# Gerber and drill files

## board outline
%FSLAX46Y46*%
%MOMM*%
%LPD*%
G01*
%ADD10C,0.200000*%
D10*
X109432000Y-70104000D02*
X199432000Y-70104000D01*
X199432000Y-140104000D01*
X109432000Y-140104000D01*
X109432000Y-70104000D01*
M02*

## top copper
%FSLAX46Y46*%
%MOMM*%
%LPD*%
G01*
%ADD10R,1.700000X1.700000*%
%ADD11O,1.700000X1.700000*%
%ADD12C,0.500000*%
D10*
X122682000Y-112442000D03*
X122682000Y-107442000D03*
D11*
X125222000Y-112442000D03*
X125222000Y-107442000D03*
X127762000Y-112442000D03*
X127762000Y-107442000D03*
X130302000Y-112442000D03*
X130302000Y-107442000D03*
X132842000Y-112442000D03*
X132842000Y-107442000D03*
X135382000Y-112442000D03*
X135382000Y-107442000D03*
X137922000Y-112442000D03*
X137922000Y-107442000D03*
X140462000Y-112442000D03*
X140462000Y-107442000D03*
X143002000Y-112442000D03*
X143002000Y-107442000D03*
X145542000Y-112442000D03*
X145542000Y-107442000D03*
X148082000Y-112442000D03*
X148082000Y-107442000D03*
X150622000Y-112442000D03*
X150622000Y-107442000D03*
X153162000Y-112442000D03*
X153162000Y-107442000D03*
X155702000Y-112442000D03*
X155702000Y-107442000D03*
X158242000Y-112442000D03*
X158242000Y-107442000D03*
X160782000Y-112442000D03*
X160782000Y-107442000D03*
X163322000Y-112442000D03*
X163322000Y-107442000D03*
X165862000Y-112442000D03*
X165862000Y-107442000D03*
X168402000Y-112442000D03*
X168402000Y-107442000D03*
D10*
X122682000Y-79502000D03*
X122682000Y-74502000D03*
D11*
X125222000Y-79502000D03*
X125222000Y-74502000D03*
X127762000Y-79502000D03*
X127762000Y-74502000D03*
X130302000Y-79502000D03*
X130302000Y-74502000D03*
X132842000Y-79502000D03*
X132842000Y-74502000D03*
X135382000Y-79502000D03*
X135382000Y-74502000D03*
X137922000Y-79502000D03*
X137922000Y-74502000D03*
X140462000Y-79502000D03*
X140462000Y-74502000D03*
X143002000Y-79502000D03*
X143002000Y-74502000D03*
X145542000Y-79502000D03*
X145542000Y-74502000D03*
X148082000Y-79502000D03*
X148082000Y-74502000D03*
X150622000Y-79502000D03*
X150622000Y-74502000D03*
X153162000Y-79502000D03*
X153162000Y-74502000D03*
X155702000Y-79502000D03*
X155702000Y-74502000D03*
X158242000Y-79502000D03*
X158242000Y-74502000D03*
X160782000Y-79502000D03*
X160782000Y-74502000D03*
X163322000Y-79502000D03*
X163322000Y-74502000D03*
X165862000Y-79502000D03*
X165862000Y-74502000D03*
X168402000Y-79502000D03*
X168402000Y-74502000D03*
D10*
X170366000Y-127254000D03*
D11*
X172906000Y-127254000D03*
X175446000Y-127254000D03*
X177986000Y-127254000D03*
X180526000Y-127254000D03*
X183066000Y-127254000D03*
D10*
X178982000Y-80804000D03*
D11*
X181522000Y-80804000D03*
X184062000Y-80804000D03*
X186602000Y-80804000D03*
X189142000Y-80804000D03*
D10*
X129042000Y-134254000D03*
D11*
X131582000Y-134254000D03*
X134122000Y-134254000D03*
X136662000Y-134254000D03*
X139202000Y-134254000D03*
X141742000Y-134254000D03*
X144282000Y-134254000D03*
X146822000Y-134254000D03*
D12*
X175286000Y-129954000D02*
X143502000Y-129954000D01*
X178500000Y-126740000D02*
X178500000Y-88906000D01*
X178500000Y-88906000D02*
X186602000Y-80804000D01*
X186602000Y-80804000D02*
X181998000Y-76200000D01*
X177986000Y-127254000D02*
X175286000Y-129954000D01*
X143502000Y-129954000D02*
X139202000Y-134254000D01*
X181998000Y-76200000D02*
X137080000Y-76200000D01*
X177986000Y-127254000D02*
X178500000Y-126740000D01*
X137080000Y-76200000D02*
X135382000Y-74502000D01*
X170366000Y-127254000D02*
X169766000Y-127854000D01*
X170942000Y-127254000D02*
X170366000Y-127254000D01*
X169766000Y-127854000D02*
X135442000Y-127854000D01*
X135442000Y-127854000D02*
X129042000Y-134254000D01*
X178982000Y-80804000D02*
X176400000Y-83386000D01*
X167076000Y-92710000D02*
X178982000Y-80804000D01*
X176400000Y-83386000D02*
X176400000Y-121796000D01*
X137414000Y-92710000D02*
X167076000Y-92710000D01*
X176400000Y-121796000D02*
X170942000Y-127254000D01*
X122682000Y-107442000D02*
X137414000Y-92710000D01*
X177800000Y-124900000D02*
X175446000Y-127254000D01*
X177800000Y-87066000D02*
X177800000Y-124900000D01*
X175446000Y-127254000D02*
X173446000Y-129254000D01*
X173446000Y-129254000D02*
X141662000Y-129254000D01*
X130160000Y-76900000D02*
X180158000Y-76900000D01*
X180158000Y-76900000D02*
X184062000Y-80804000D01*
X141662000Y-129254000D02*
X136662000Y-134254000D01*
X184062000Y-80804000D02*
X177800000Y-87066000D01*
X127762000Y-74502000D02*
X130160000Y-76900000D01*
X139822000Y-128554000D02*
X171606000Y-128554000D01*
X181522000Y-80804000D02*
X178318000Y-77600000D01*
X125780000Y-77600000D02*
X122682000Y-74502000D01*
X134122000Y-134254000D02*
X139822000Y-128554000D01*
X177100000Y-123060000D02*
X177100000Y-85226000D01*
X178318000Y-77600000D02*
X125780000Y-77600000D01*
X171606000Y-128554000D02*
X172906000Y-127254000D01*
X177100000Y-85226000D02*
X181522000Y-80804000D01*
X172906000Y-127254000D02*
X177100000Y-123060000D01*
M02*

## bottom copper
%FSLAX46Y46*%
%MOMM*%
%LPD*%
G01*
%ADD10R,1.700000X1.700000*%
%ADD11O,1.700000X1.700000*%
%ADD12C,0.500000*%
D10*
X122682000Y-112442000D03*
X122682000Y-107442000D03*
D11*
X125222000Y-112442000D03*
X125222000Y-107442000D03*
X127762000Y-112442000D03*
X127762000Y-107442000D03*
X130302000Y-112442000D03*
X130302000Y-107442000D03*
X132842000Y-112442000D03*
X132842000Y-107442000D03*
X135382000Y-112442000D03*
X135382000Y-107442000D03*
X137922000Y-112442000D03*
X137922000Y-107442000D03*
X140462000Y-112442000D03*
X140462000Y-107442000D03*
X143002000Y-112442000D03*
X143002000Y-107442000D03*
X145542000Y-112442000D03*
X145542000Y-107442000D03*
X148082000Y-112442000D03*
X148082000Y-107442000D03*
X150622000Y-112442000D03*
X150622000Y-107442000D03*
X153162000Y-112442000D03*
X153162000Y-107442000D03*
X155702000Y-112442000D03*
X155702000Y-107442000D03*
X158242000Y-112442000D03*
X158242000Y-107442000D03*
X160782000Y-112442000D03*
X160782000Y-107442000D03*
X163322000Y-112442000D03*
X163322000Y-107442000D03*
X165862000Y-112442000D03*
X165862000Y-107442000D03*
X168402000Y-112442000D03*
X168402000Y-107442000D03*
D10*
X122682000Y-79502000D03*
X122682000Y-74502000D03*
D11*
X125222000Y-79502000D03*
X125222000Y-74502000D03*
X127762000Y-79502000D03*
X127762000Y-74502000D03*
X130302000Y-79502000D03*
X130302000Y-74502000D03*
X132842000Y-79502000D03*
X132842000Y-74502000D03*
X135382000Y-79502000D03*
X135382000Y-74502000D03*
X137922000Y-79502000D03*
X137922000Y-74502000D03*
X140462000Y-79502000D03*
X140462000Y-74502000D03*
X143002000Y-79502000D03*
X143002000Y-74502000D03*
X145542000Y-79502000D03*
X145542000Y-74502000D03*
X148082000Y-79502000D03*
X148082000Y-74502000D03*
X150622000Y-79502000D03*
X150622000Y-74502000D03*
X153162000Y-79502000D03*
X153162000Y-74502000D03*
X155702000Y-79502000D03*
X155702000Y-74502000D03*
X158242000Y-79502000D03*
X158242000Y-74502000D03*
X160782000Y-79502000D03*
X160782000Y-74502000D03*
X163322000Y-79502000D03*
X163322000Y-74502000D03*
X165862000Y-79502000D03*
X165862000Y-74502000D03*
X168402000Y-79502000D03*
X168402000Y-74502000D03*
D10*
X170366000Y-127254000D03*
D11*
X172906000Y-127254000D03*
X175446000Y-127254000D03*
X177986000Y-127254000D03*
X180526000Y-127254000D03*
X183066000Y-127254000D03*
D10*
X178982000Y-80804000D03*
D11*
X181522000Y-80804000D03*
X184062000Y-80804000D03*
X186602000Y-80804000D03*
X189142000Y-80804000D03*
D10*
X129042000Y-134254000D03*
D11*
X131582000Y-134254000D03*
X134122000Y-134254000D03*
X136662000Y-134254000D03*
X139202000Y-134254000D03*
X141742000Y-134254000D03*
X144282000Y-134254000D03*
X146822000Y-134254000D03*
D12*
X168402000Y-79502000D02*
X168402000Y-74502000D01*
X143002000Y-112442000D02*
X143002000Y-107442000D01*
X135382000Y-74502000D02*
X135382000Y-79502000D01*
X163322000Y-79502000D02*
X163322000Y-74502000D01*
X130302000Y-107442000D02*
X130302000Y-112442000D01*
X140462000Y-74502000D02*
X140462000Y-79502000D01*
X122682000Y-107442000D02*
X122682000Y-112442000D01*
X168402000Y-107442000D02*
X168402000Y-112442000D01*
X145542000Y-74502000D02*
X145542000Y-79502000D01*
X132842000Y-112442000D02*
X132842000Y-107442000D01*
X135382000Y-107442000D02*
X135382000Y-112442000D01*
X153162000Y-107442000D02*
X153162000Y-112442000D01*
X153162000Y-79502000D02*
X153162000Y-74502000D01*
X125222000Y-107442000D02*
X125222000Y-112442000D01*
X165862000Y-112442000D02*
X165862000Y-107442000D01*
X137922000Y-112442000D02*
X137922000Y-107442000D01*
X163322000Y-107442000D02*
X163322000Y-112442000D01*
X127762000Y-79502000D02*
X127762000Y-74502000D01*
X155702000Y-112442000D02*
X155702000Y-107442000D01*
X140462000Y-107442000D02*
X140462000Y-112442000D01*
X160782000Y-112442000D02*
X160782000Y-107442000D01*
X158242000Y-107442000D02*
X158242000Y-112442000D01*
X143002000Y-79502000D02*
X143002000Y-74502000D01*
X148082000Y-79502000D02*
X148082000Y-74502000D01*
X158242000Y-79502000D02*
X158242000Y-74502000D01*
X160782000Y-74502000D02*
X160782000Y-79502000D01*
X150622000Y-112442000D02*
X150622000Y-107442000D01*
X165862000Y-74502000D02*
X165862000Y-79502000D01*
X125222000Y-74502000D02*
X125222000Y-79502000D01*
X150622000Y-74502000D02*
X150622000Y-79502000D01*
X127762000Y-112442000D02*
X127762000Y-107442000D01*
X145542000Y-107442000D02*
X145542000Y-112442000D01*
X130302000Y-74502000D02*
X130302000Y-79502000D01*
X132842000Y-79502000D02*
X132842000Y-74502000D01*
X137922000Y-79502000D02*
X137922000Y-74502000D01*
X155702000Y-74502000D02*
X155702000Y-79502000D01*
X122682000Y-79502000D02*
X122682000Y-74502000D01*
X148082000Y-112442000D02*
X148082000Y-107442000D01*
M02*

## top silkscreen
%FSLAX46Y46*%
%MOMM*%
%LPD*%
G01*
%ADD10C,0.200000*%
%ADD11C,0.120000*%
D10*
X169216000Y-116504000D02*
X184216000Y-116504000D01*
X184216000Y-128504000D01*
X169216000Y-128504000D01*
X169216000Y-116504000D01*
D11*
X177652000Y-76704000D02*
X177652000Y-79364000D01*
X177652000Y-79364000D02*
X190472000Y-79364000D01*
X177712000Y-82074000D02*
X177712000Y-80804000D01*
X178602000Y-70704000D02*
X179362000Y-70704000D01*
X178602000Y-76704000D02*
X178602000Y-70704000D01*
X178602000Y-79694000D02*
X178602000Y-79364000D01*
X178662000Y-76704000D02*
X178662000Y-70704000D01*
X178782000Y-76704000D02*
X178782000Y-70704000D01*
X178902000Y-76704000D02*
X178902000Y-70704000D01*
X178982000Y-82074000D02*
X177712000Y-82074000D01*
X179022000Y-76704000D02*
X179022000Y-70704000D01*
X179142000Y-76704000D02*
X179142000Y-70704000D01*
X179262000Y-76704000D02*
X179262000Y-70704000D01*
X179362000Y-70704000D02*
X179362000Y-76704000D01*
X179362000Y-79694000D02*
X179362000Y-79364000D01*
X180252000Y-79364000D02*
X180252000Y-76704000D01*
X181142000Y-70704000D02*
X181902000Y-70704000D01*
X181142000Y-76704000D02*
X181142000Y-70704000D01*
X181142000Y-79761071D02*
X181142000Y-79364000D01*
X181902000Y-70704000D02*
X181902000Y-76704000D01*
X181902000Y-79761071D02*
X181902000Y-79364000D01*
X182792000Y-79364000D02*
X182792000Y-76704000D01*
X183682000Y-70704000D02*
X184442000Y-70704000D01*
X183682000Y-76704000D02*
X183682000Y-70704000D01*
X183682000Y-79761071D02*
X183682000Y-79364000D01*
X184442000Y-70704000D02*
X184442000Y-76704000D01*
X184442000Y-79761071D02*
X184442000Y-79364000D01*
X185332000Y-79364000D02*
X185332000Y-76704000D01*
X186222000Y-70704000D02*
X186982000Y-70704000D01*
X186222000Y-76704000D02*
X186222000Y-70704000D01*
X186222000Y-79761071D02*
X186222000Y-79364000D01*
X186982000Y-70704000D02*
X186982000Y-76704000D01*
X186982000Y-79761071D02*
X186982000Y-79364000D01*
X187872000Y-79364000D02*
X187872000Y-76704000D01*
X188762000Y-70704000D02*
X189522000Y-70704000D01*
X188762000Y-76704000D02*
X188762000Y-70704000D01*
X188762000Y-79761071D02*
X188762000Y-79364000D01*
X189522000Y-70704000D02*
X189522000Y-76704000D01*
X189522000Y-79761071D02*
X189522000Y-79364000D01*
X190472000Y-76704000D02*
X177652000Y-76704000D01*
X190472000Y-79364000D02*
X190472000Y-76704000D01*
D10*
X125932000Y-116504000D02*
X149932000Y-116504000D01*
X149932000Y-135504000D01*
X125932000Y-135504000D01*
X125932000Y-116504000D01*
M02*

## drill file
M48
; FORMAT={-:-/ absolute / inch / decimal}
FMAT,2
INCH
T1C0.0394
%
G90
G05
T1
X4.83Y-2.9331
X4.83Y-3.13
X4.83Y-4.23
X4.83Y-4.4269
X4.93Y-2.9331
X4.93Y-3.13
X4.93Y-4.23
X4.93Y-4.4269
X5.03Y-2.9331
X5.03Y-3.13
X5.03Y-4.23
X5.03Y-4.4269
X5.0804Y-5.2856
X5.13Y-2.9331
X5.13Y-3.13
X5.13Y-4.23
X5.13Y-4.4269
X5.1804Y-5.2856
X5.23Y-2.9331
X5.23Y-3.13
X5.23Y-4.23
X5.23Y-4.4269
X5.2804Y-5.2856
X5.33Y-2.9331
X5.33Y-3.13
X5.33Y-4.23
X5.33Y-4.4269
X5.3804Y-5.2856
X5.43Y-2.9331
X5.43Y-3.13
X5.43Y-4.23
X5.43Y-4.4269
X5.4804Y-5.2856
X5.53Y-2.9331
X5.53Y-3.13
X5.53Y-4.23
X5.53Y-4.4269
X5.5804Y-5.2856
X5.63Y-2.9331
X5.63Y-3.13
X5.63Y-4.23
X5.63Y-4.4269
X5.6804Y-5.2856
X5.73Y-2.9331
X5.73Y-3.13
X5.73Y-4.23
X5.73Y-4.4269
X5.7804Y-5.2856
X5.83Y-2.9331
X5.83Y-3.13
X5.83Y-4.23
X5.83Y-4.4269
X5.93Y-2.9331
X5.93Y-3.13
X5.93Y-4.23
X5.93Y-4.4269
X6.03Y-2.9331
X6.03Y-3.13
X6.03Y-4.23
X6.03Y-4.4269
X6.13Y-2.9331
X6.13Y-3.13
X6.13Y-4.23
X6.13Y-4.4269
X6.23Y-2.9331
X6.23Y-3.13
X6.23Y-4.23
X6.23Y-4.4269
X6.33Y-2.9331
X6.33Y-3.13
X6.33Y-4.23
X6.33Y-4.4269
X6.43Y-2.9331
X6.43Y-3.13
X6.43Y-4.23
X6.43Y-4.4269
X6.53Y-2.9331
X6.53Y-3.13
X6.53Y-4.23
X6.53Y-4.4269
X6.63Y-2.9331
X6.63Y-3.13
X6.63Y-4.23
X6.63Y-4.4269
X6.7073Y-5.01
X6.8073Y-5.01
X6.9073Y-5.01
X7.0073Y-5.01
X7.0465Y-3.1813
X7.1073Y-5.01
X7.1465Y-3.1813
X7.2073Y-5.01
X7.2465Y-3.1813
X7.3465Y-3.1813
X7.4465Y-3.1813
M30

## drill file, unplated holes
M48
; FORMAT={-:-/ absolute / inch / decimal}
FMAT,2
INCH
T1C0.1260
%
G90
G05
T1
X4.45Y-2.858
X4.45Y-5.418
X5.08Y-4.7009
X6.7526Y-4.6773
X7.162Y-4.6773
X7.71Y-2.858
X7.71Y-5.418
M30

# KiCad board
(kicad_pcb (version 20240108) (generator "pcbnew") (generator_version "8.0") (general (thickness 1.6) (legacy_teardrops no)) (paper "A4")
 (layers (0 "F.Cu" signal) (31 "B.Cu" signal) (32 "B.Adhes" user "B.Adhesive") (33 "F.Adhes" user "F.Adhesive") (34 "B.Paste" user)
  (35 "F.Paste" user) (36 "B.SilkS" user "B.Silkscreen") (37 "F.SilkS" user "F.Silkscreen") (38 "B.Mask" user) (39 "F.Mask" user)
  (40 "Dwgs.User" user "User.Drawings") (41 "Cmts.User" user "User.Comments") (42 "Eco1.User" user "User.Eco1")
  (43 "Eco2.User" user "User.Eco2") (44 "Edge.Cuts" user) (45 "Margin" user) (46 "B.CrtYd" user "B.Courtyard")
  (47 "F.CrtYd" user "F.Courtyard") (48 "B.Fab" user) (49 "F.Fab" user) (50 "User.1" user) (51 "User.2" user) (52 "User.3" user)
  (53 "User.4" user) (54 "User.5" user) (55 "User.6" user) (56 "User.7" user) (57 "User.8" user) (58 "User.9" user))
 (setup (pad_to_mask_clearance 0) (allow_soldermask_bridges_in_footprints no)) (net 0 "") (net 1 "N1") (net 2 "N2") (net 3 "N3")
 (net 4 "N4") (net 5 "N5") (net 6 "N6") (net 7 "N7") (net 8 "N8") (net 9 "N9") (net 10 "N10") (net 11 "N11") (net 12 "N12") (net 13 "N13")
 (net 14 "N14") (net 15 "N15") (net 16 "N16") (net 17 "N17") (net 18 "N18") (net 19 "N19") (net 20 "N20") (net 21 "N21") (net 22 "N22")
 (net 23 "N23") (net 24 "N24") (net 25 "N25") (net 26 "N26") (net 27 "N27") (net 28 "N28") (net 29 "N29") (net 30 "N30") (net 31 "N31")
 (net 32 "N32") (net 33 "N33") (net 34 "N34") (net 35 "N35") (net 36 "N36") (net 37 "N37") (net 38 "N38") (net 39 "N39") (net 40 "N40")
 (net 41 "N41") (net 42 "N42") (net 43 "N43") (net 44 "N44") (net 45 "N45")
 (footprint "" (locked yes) (layer "F.Cu") (at 113.03 72.592)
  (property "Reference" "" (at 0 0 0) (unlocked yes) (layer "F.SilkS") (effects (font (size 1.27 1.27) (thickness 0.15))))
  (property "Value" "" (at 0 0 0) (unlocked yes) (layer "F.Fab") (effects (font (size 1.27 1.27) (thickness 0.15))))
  (pad "" np_thru_hole circle (at 0 0) (size 3.2 3.2) (drill 3.2) (layers "F&B.Cu" "*.Mask")))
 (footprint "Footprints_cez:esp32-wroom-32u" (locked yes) (layer "F.Cu") (at 134.864 94.742 90)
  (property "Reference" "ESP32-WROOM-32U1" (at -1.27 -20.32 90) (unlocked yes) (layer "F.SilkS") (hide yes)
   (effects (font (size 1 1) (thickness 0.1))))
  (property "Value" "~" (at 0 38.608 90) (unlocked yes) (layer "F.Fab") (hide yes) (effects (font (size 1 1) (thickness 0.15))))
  (pad "1" thru_hole rect (at -17.7 -12.182 90) (size 1.7 1.7) (drill 1) (layers "*.Cu" "*.Mask") (remove_unused_layers no) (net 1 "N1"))
  (pad "1" thru_hole rect (at -12.7 -12.182 90) (size 1.7 1.7) (drill 1) (layers "*.Cu" "*.Mask") (remove_unused_layers no) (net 1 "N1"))
  (pad "2" thru_hole oval (at -17.7 -9.642 90) (size 1.7 1.7) (drill 1) (layers "*.Cu" "*.Mask") (remove_unused_layers no) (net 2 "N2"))
  (pad "2" thru_hole oval (at -12.7 -9.642 90) (size 1.7 1.7) (drill 1) (layers "*.Cu" "*.Mask") (remove_unused_layers no) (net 2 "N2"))
  (pad "3" thru_hole oval (at -17.7 -7.102 90) (size 1.7 1.7) (drill 1) (layers "*.Cu" "*.Mask") (remove_unused_layers no) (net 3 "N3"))
  (pad "3" thru_hole oval (at -12.7 -7.102 90) (size 1.7 1.7) (drill 1) (layers "*.Cu" "*.Mask") (remove_unused_layers no) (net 3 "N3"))
  (pad "4" thru_hole oval (at -17.7 -4.562 90) (size 1.7 1.7) (drill 1) (layers "*.Cu" "*.Mask") (remove_unused_layers no) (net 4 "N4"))
  (pad "4" thru_hole oval (at -12.7 -4.562 90) (size 1.7 1.7) (drill 1) (layers "*.Cu" "*.Mask") (remove_unused_layers no) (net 4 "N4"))
  (pad "5" thru_hole oval (at -17.7 -2.022 90) (size 1.7 1.7) (drill 1) (layers "*.Cu" "*.Mask") (remove_unused_layers no) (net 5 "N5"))
  (pad "5" thru_hole oval (at -12.7 -2.022 90) (size 1.7 1.7) (drill 1) (layers "*.Cu" "*.Mask") (remove_unused_layers no) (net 5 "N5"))
  (pad "6" thru_hole oval (at -17.7 0.518 90) (size 1.7 1.7) (drill 1) (layers "*.Cu" "*.Mask") (remove_unused_layers no) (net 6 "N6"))
  (pad "6" thru_hole oval (at -12.7 0.518 90) (size 1.7 1.7) (drill 1) (layers "*.Cu" "*.Mask") (remove_unused_layers no) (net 6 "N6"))
  (pad "7" thru_hole oval (at -17.7 3.058 90) (size 1.7 1.7) (drill 1) (layers "*.Cu" "*.Mask") (remove_unused_layers no) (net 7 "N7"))
  (pad "7" thru_hole oval (at -12.7 3.058 90) (size 1.7 1.7) (drill 1) (layers "*.Cu" "*.Mask") (remove_unused_layers no) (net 7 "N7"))
  (pad "8" thru_hole oval (at -17.7 5.598 90) (size 1.7 1.7) (drill 1) (layers "*.Cu" "*.Mask") (remove_unused_layers no) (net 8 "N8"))
  (pad "8" thru_hole oval (at -12.7 5.598 90) (size 1.7 1.7) (drill 1) (layers "*.Cu" "*.Mask") (remove_unused_layers no) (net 8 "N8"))
  (pad "9" thru_hole oval (at -17.7 8.138 90) (size 1.7 1.7) (drill 1) (layers "*.Cu" "*.Mask") (remove_unused_layers no) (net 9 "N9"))
  (pad "9" thru_hole oval (at -12.7 8.138 90) (size 1.7 1.7) (drill 1) (layers "*.Cu" "*.Mask") (remove_unused_layers no) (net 9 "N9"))
  (pad "10" thru_hole oval (at -17.7 10.678 90) (size 1.7 1.7) (drill 1) (layers "*.Cu" "*.Mask") (remove_unused_layers no) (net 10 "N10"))
  (pad "10" thru_hole oval (at -12.7 10.678 90) (size 1.7 1.7) (drill 1) (layers "*.Cu" "*.Mask") (remove_unused_layers no) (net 10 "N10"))
  (pad "11" thru_hole oval (at -17.7 13.218 90) (size 1.7 1.7) (drill 1) (layers "*.Cu" "*.Mask") (remove_unused_layers no) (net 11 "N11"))
  (pad "11" thru_hole oval (at -12.7 13.218 90) (size 1.7 1.7) (drill 1) (layers "*.Cu" "*.Mask") (remove_unused_layers no) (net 11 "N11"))
  (pad "12" thru_hole oval (at -17.7 15.758 90) (size 1.7 1.7) (drill 1) (layers "*.Cu" "*.Mask") (remove_unused_layers no) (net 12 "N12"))
  (pad "12" thru_hole oval (at -12.7 15.758 90) (size 1.7 1.7) (drill 1) (layers "*.Cu" "*.Mask") (remove_unused_layers no) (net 12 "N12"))
  (pad "13" thru_hole oval (at -17.7 18.298 90) (size 1.7 1.7) (drill 1) (layers "*.Cu" "*.Mask") (remove_unused_layers no) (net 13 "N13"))
  (pad "13" thru_hole oval (at -12.7 18.298 90) (size 1.7 1.7) (drill 1) (layers "*.Cu" "*.Mask") (remove_unused_layers no) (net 13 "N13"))
  (pad "14" thru_hole oval (at -17.7 20.838 90) (size 1.7 1.7) (drill 1) (layers "*.Cu" "*.Mask") (remove_unused_layers no) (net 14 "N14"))
  (pad "14" thru_hole oval (at -12.7 20.838 90) (size 1.7 1.7) (drill 1) (layers "*.Cu" "*.Mask") (remove_unused_layers no) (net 14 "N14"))
  (pad "15" thru_hole oval (at -17.7 23.378 90) (size 1.7 1.7) (drill 1) (layers "*.Cu" "*.Mask") (remove_unused_layers no) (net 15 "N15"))
  (pad "15" thru_hole oval (at -12.7 23.378 90) (size 1.7 1.7) (drill 1) (layers "*.Cu" "*.Mask") (remove_unused_layers no) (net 15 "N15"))
  (pad "16" thru_hole oval (at -17.7 25.918 90) (size 1.7 1.7) (drill 1) (layers "*.Cu" "*.Mask") (remove_unused_layers no) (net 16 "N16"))
  (pad "16" thru_hole oval (at -12.7 25.918 90) (size 1.7 1.7) (drill 1) (layers "*.Cu" "*.Mask") (remove_unused_layers no) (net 16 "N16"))
  (pad "17" thru_hole oval (at -17.7 28.458 90) (size 1.7 1.7) (drill 1) (layers "*.Cu" "*.Mask") (remove_unused_layers no) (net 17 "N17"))
  (pad "17" thru_hole oval (at -12.7 28.458 90) (size 1.7 1.7) (drill 1) (layers "*.Cu" "*.Mask") (remove_unused_layers no) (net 17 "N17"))
  (pad "18" thru_hole oval (at -17.7 30.998 90) (size 1.7 1.7) (drill 1) (layers "*.Cu" "*.Mask") (remove_unused_layers no) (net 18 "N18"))
  (pad "18" thru_hole oval (at -12.7 30.998 90) (size 1.7 1.7) (drill 1) (layers "*.Cu" "*.Mask") (remove_unused_layers no) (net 18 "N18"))
  (pad "19" thru_hole oval (at -17.7 33.538 90) (size 1.7 1.7) (drill 1) (layers "*.Cu" "*.Mask") (remove_unused_layers no) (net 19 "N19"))
  (pad "19" thru_hole oval (at -12.7 33.538 90) (size 1.7 1.7) (drill 1) (layers "*.Cu" "*.Mask") (remove_unused_layers no) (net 19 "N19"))
  (pad "20" thru_hole rect (at 15.24 -12.182 90) (size 1.7 1.7) (drill 1) (layers "*.Cu" "*.Mask") (remove_unused_layers no) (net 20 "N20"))
  (pad "20" thru_hole rect (at 20.24 -12.182 90) (size 1.7 1.7) (drill 1) (layers "*.Cu" "*.Mask") (remove_unused_layers no) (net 20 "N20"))
  (pad "21" thru_hole oval (at 15.24 -9.642 90) (size 1.7 1.7) (drill 1) (layers "*.Cu" "*.Mask") (remove_unused_layers no) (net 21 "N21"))
  (pad "21" thru_hole oval (at 20.24 -9.642 90) (size 1.7 1.7) (drill 1) (layers "*.Cu" "*.Mask") (remove_unused_layers no) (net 21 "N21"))
  (pad "22" thru_hole oval (at 15.24 -7.102 90) (size 1.7 1.7) (drill 1) (layers "*.Cu" "*.Mask") (remove_unused_layers no) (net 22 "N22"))
  (pad "22" thru_hole oval (at 20.24 -7.102 90) (size 1.7 1.7) (drill 1) (layers "*.Cu" "*.Mask") (remove_unused_layers no) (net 22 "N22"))
  (pad "23" thru_hole oval (at 15.24 -4.562 90) (size 1.7 1.7) (drill 1) (layers "*.Cu" "*.Mask") (remove_unused_layers no) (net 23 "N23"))
  (pad "23" thru_hole oval (at 20.24 -4.562 90) (size 1.7 1.7) (drill 1) (layers "*.Cu" "*.Mask") (remove_unused_layers no) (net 23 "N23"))
  (pad "24" thru_hole oval (at 15.24 -2.022 90) (size 1.7 1.7) (drill 1) (layers "*.Cu" "*.Mask") (remove_unused_layers no) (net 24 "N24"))
  (pad "24" thru_hole oval (at 20.24 -2.022 90) (size 1.7 1.7) (drill 1) (layers "*.Cu" "*.Mask") (remove_unused_layers no) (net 24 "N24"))
  (pad "25" thru_hole oval (at 15.24 0.518 90) (size 1.7 1.7) (drill 1) (layers "*.Cu" "*.Mask") (remove_unused_layers no) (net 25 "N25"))
  (pad "25" thru_hole oval (at 20.24 0.518 90) (size 1.7 1.7) (drill 1) (layers "*.Cu" "*.Mask") (remove_unused_layers no) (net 25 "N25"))
  (pad "26" thru_hole oval (at 15.24 3.058 90) (size 1.7 1.7) (drill 1) (layers "*.Cu" "*.Mask") (remove_unused_layers no) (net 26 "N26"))
  (pad "26" thru_hole oval (at 20.24 3.058 90) (size 1.7 1.7) (drill 1) (layers "*.Cu" "*.Mask") (remove_unused_layers no) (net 26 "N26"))
  (pad "27" thru_hole oval (at 15.24 5.598 90) (size 1.7 1.7) (drill 1) (layers "*.Cu" "*.Mask") (remove_unused_layers no) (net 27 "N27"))
  (pad "27" thru_hole oval (at 20.24 5.598 90) (size 1.7 1.7) (drill 1) (layers "*.Cu" "*.Mask") (remove_unused_layers no) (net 27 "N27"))
  (pad "28" thru_hole oval (at 15.24 8.138 90) (size 1.7 1.7) (drill 1) (layers "*.Cu" "*.Mask") (remove_unused_layers no) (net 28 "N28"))
  (pad "28" thru_hole oval (at 20.24 8.138 90) (size 1.7 1.7) (drill 1) (layers "*.Cu" "*.Mask") (remove_unused_layers no) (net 28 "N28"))
  (pad "29" thru_hole oval (at 15.24 10.678 90) (size 1.7 1.7) (drill 1) (layers "*.Cu" "*.Mask") (remove_unused_layers no) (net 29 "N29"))
  (pad "29" thru_hole oval (at 20.24 10.678 90) (size 1.7 1.7) (drill 1) (layers "*.Cu" "*.Mask") (remove_unused_layers no) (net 29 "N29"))
  (pad "30" thru_hole oval (at 15.24 13.218 90) (size 1.7 1.7) (drill 1) (layers "*.Cu" "*.Mask") (remove_unused_layers no) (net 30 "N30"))
  (pad "30" thru_hole oval (at 20.24 13.218 90) (size 1.7 1.7) (drill 1) (layers "*.Cu" "*.Mask") (remove_unused_layers no) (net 30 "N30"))
  (pad "31" thru_hole oval (at 15.24 15.758 90) (size 1.7 1.7) (drill 1) (layers "*.Cu" "*.Mask") (remove_unused_layers no) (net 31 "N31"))
  (pad "31" thru_hole oval (at 20.24 15.758 90) (size 1.7 1.7) (drill 1) (layers "*.Cu" "*.Mask") (remove_unused_layers no) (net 31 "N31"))
  (pad "32" thru_hole oval (at 15.24 18.298 90) (size 1.7 1.7) (drill 1) (layers "*.Cu" "*.Mask") (remove_unused_layers no) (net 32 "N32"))
  (pad "32" thru_hole oval (at 20.24 18.298 90) (size 1.7 1.7) (drill 1) (layers "*.Cu" "*.Mask") (remove_unused_layers no) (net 32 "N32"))
  (pad "33" thru_hole oval (at 15.24 20.838 90) (size 1.7 1.7) (drill 1) (layers "*.Cu" "*.Mask") (remove_unused_layers no) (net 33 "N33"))
  (pad "33" thru_hole oval (at 20.24 20.838 90) (size 1.7 1.7) (drill 1) (layers "*.Cu" "*.Mask") (remove_unused_layers no) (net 33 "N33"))
  (pad "34" thru_hole oval (at 15.24 23.378 90) (size 1.7 1.7) (drill 1) (layers "*.Cu" "*.Mask") (remove_unused_layers no) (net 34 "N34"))
  (pad "34" thru_hole oval (at 20.24 23.378 90) (size 1.7 1.7) (drill 1) (layers "*.Cu" "*.Mask") (remove_unused_layers no) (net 34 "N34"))
  (pad "35" thru_hole oval (at 15.24 25.918 90) (size 1.7 1.7) (drill 1) (layers "*.Cu" "*.Mask") (remove_unused_layers no) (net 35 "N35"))
  (pad "35" thru_hole oval (at 20.24 25.918 90) (size 1.7 1.7) (drill 1) (layers "*.Cu" "*.Mask") (remove_unused_layers no) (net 35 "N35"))
  (pad "36" thru_hole oval (at 15.24 28.458 90) (size 1.7 1.7) (drill 1) (layers "*.Cu" "*.Mask") (remove_unused_layers no) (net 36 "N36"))
  (pad "36" thru_hole oval (at 20.24 28.458 90) (size 1.7 1.7) (drill 1) (layers "*.Cu" "*.Mask") (remove_unused_layers no) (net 36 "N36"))
  (pad "37" thru_hole oval (at 15.24 30.998 90) (size 1.7 1.7) (drill 1) (layers "*.Cu" "*.Mask") (remove_unused_layers no) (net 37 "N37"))
  (pad "37" thru_hole oval (at 20.24 30.998 90) (size 1.7 1.7) (drill 1) (layers "*.Cu" "*.Mask") (remove_unused_layers no) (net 37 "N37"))
  (pad "38" thru_hole oval (at 15.24 33.538 90) (size 1.7 1.7) (drill 1) (layers "*.Cu" "*.Mask") (remove_unused_layers no) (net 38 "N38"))
  (pad "38" thru_hole oval (at 20.24 33.538 90) (size 1.7 1.7) (drill 1) (layers "*.Cu" "*.Mask") (remove_unused_layers no) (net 38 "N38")))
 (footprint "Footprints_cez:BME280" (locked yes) (layer "F.Cu") (at 178.755 110.185)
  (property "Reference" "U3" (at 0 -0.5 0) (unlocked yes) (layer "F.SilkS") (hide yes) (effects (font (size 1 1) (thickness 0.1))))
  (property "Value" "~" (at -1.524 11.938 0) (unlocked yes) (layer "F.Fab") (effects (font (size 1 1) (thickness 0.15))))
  (fp_rect (start -9.539 6.319) (end 5.461 18.319) (stroke (width 0.2) (type default)) (fill none) (layer "F.SilkS"))
  (pad "" np_thru_hole circle (at -7.239 8.619) (size 3.2 3.2) (drill 3.2) (layers "F&B.Cu" "*.Mask"))
  (pad "" np_thru_hole circle (at 3.161 8.619) (size 3.2 3.2) (drill 3.2) (layers "F&B.Cu" "*.Mask"))
  (pad "1" thru_hole rect (at -8.389 17.069 90) (size 1.7 1.7) (drill 1) (layers "*.Cu" "*.Mask") (remove_unused_layers no) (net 1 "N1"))
  (pad "2" thru_hole oval (at -5.849 17.069 90) (size 1.7 1.7) (drill 1) (layers "*.Cu" "*.Mask") (remove_unused_layers no) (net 20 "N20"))
  (pad "3" thru_hole oval (at -3.309 17.069 90) (size 1.7 1.7) (drill 1) (layers "*.Cu" "*.Mask") (remove_unused_layers no) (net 22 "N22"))
  (pad "4" thru_hole oval (at -0.769 17.069 90) (size 1.7 1.7) (drill 1) (layers "*.Cu" "*.Mask") (remove_unused_layers no) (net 25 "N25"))
  (pad "5" thru_hole oval (at 1.771 17.069 90) (size 1.7 1.7) (drill 1) (layers "*.Cu" "*.Mask") (remove_unused_layers no) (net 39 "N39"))
  (pad "6" thru_hole oval (at 4.311 17.069 90) (size 1.7 1.7) (drill 1) (layers "*.Cu" "*.Mask") (remove_unused_layers no) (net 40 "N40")))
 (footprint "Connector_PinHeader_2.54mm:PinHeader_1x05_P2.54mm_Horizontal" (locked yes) (layer "F.Cu") (at 178.982 80.804 90)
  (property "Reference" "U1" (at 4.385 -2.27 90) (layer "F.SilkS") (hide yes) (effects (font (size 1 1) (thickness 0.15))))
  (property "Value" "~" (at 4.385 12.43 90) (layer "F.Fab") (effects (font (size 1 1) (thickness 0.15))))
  (fp_line (start 4.1 -1.33) (end 1.44 -1.33) (stroke (width 0.12) (type solid)) (layer "F.SilkS"))
  (fp_line (start 1.44 -1.33) (end 1.44 11.49) (stroke (width 0.12) (type solid)) (layer "F.SilkS"))
  (fp_line (start -1.27 -1.27) (end 0 -1.27) (stroke (width 0.12) (type solid)) (layer "F.SilkS"))
  (fp_line (start 10.1 -0.38) (end 10.1 0.38) (stroke (width 0.12) (type solid)) (layer "F.SilkS"))
  (fp_line (start 4.1 -0.38) (end 10.1 -0.38) (stroke (width 0.12) (type solid)) (layer "F.SilkS"))
  (fp_line (start 1.11 -0.38) (end 1.44 -0.38) (stroke (width 0.12) (type solid)) (layer "F.SilkS"))
  (fp_line (start 4.1 -0.32) (end 10.1 -0.32) (stroke (width 0.12) (type solid)) (layer "F.SilkS"))
  (fp_line (start 4.1 -0.2) (end 10.1 -0.2) (stroke (width 0.12) (type solid)) (layer "F.SilkS"))
  (fp_line (start 4.1 -0.08) (end 10.1 -0.08) (stroke (width 0.12) (type solid)) (layer "F.SilkS"))
  (fp_line (start -1.27 0) (end -1.27 -1.27) (stroke (width 0.12) (type solid)) (layer "F.SilkS"))
  (fp_line (start 4.1 0.04) (end 10.1 0.04) (stroke (width 0.12) (type solid)) (layer "F.SilkS"))
  (fp_line (start 4.1 0.16) (end 10.1 0.16) (stroke (width 0.12) (type solid)) (layer "F.SilkS"))
  (fp_line (start 4.1 0.28) (end 10.1 0.28) (stroke (width 0.12) (type solid)) (layer "F.SilkS"))
  (fp_line (start 10.1 0.38) (end 4.1 0.38) (stroke (width 0.12) (type solid)) (layer "F.SilkS"))
  (fp_line (start 1.11 0.38) (end 1.44 0.38) (stroke (width 0.12) (type solid)) (layer "F.SilkS"))
  (fp_line (start 1.44 1.27) (end 4.1 1.27) (stroke (width 0.12) (type solid)) (layer "F.SilkS"))
  (fp_line (start 10.1 2.16) (end 10.1 2.92) (stroke (width 0.12) (type solid)) (layer "F.SilkS"))
  (fp_line (start 4.1 2.16) (end 10.1 2.16) (stroke (width 0.12) (type solid)) (layer "F.SilkS"))
  (fp_line (start 1.042929 2.16) (end 1.44 2.16) (stroke (width 0.12) (type solid)) (layer "F.SilkS"))
  (fp_line (start 10.1 2.92) (end 4.1 2.92) (stroke (width 0.12) (type solid)) (layer "F.SilkS"))
  (fp_line (start 1.042929 2.92) (end 1.44 2.92) (stroke (width 0.12) (type solid)) (layer "F.SilkS"))
  (fp_line (start 1.44 3.81) (end 4.1 3.81) (stroke (width 0.12) (type solid)) (layer "F.SilkS"))
  (fp_line (start 10.1 4.7) (end 10.1 5.46) (stroke (width 0.12) (type solid)) (layer "F.SilkS"))
  (fp_line (start 4.1 4.7) (end 10.1 4.7) (stroke (width 0.12) (type solid)) (layer "F.SilkS"))
  (fp_line (start 1.042929 4.7) (end 1.44 4.7) (stroke (width 0.12) (type solid)) (layer "F.SilkS"))
  (fp_line (start 10.1 5.46) (end 4.1 5.46) (stroke (width 0.12) (type solid)) (layer "F.SilkS"))
  (fp_line (start 1.042929 5.46) (end 1.44 5.46) (stroke (width 0.12) (type solid)) (layer "F.SilkS"))
  (fp_line (start 1.44 6.35) (end 4.1 6.35) (stroke (width 0.12) (type solid)) (layer "F.SilkS"))
  (fp_line (start 10.1 7.24) (end 10.1 8) (stroke (width 0.12) (type solid)) (layer "F.SilkS"))
  (fp_line (start 4.1 7.24) (end 10.1 7.24) (stroke (width 0.12) (type solid)) (layer "F.SilkS"))
  (fp_line (start 1.042929 7.24) (end 1.44 7.24) (stroke (width 0.12) (type solid)) (layer "F.SilkS"))
  (fp_line (start 10.1 8) (end 4.1 8) (stroke (width 0.12) (type solid)) (layer "F.SilkS"))
  (fp_line (start 1.042929 8) (end 1.44 8) (stroke (width 0.12) (type solid)) (layer "F.SilkS"))
  (fp_line (start 1.44 8.89) (end 4.1 8.89) (stroke (width 0.12) (type solid)) (layer "F.SilkS"))
  (fp_line (start 10.1 9.78) (end 10.1 10.54) (stroke (width 0.12) (type solid)) (layer "F.SilkS"))
  (fp_line (start 4.1 9.78) (end 10.1 9.78) (stroke (width 0.12) (type solid)) (layer "F.SilkS"))
  (fp_line (start 1.042929 9.78) (end 1.44 9.78) (stroke (width 0.12) (type solid)) (layer "F.SilkS"))
  (fp_line (start 10.1 10.54) (end 4.1 10.54) (stroke (width 0.12) (type solid)) (layer "F.SilkS"))
  (fp_line (start 1.042929 10.54) (end 1.44 10.54) (stroke (width 0.12) (type solid)) (layer "F.SilkS"))
  (fp_line (start 4.1 11.49) (end 4.1 -1.33) (stroke (width 0.12) (type solid)) (layer "F.SilkS"))
  (fp_line (start 1.44 11.49) (end 4.1 11.49) (stroke (width 0.12) (type solid)) (layer "F.SilkS"))
  (pad "1" thru_hole rect (at 0 0 90) (size 1.7 1.7) (drill 1) (layers "*.Cu" "*.Mask") (remove_unused_layers no) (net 1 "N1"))
  (pad "2" thru_hole oval (at 0 2.54 90) (size 1.7 1.7) (drill 1) (layers "*.Cu" "*.Mask") (remove_unused_layers no) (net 20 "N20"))
  (pad "3" thru_hole oval (at 0 5.08 90) (size 1.7 1.7) (drill 1) (layers "*.Cu" "*.Mask") (remove_unused_layers no) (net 22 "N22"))
  (pad "4" thru_hole oval (at 0 7.62 90) (size 1.7 1.7) (drill 1) (layers "*.Cu" "*.Mask") (remove_unused_layers no) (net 25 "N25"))
  (pad "5" thru_hole oval (at 0 10.16 90) (size 1.7 1.7) (drill 1) (layers "*.Cu" "*.Mask") (remove_unused_layers no) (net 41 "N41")))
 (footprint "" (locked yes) (layer "F.Cu") (at 113.03 137.616)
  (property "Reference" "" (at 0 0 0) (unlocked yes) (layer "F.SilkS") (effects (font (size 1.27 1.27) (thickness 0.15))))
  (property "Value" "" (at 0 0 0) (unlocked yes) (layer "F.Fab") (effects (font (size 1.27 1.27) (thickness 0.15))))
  (pad "" np_thru_hole circle (at 0 0) (size 3.2 3.2) (drill 3.2) (layers "F&B.Cu" "*.Mask")))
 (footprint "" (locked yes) (layer "F.Cu") (at 195.834 137.616)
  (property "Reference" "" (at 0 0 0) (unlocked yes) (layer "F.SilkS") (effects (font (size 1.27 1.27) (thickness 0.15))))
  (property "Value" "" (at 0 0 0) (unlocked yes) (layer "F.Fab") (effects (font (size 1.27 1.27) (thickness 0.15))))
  (pad "" np_thru_hole circle (at 0 0) (size 3.2 3.2) (drill 3.2) (layers "F&B.Cu" "*.Mask")))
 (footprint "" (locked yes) (layer "F.Cu") (at 195.834 72.592)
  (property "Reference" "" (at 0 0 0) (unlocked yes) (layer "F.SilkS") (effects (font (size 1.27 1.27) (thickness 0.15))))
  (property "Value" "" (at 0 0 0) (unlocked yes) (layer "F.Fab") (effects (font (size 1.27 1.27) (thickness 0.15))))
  (pad "" np_thru_hole circle (at 0 0) (size 3.2 3.2) (drill 3.2) (layers "F&B.Cu" "*.Mask")))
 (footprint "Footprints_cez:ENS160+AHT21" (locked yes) (layer "F.Cu") (at 136.027 102.611)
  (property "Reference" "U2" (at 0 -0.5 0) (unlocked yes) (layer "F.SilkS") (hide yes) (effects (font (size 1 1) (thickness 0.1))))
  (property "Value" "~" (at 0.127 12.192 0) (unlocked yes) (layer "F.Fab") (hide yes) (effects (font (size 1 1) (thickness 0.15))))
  (fp_rect (start -10.095 13.893) (end 13.905 32.893) (stroke (width 0.2) (type default)) (fill none) (layer "F.SilkS"))
  (pad "" np_thru_hole circle (at -6.995 16.793) (size 3.2 3.2) (drill 3.2) (layers "*.Cu" "*.Mask"))
  (pad "1" thru_hole rect (at -6.985 31.643 90) (size 1.7 1.7) (drill 1) (layers "*.Cu" "*.Mask") (remove_unused_layers no) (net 1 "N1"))
  (pad "2" thru_hole oval (at -4.445 31.643 90) (size 1.7 1.7) (drill 1) (layers "*.Cu" "*.Mask") (remove_unused_layers no) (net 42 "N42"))
  (pad "3" thru_hole oval (at -1.905 31.643 90) (size 1.7 1.7) (drill 1) (layers "*.Cu" "*.Mask") (remove_unused_layers no) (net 20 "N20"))
  (pad "4" thru_hole oval (at 0.635 31.643 90) (size 1.7 1.7) (drill 1) (layers "*.Cu" "*.Mask") (remove_unused_layers no) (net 22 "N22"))
  (pad "5" thru_hole oval (at 3.175 31.643 90) (size 1.7 1.7) (drill 1) (layers "*.Cu" "*.Mask") (remove_unused_layers no) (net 25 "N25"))
  (pad "6" thru_hole oval (at 5.715 31.643 90) (size 1.7 1.7) (drill 1) (layers "*.Cu" "*.Mask") (remove_unused_layers no) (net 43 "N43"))
  (pad "7" thru_hole oval (at 8.255 31.643 90) (size 1.7 1.7) (drill 1) (layers "*.Cu" "*.Mask") (remove_unused_layers no) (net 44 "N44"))
  (pad "8" thru_hole oval (at 10.795 31.643 90) (size 1.7 1.7) (drill 1) (layers "*.Cu" "*.Mask") (remove_unused_layers no) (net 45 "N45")))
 (gr_rect (start 109.432 70.104) (end 199.432 140.104) (locked yes) (stroke (width 0.2) (type default)) (fill none) (layer "Edge.Cuts"))
 (segment (start 168.402 79.502) (end 168.402 74.502) (width 0.5) (layer "B.Cu") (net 38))
 (segment (start 143.002 112.442) (end 143.002 107.442) (width 0.5) (layer "B.Cu") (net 9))
 (segment (start 175.286 129.954) (end 143.502 129.954) (width 0.5) (layer "F.Cu") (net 25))
 (segment (start 178.5 126.74) (end 178.5 88.906) (width 0.5) (layer "F.Cu") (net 25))
 (segment (start 178.5 88.906) (end 186.602 80.804) (width 0.5) (layer "F.Cu") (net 25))
 (segment (start 186.602 80.804) (end 181.998 76.2) (width 0.5) (layer "F.Cu") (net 25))
 (segment (start 177.986 127.254) (end 175.286 129.954) (width 0.5) (layer "F.Cu") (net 25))
 (segment (start 143.502 129.954) (end 139.202 134.254) (width 0.5) (layer "F.Cu") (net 25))
 (segment (start 181.998 76.2) (end 137.08 76.2) (width 0.5) (layer "F.Cu") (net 25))
 (segment (start 177.986 127.254) (end 178.5 126.74) (width 0.5) (layer "F.Cu") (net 25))
 (segment (start 137.08 76.2) (end 135.382 74.502) (width 0.5) (layer "F.Cu") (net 25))
 (segment (start 135.382 74.502) (end 135.382 79.502) (width 0.5) (layer "B.Cu") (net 25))
 (segment (start 163.322 79.502) (end 163.322 74.502) (width 0.5) (layer "B.Cu") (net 36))
 (segment (start 130.302 107.442) (end 130.302 112.442) (width 0.5) (layer "B.Cu") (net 4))
 (segment (start 140.462 74.502) (end 140.462 79.502) (width 0.5) (layer "B.Cu") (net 27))
 (segment (start 170.366 127.254) (end 169.766 127.854) (width 0.5) (layer "F.Cu") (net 1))
 (segment (start 170.942 127.254) (end 170.366 127.254) (width 0.5) (layer "F.Cu") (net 1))
 (segment (start 169.766 127.854) (end 135.442 127.854) (width 0.5) (layer "F.Cu") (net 1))
 (segment (start 135.442 127.854) (end 129.042 134.254) (width 0.5) (layer "F.Cu") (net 1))
 (segment (start 178.982 80.804) (end 176.4 83.386) (width 0.5) (layer "F.Cu") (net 1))
 (segment (start 167.076 92.71) (end 178.982 80.804) (width 0.5) (layer "F.Cu") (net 1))
 (segment (start 176.4 83.386) (end 176.4 121.796) (width 0.5) (layer "F.Cu") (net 1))
 (segment (start 137.414 92.71) (end 167.076 92.71) (width 0.5) (layer "F.Cu") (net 1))
 (segment (start 176.4 121.796) (end 170.942 127.254) (width 0.5) (layer "F.Cu") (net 1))
 (segment (start 122.682 107.442) (end 137.414 92.71) (width 0.5) (layer "F.Cu") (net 1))
 (segment (start 122.682 107.442) (end 122.682 112.442) (width 0.5) (layer "B.Cu") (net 1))
 (segment (start 168.402 107.442) (end 168.402 112.442) (width 0.5) (layer "B.Cu") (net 19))
 (segment (start 145.542 74.502) (end 145.542 79.502) (width 0.5) (layer "B.Cu") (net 29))
 (segment (start 132.842 112.442) (end 132.842 107.442) (width 0.5) (layer "B.Cu") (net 5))
 (segment (start 135.382 107.442) (end 135.382 112.442) (width 0.5) (layer "B.Cu") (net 6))
 (segment (start 153.162 107.442) (end 153.162 112.442) (width 0.5) (layer "B.Cu") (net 13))
 (segment (start 153.162 79.502) (end 153.162 74.502) (width 0.5) (layer "B.Cu") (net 32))
 (segment (start 125.222 107.442) (end 125.222 112.442) (width 0.5) (layer "B.Cu") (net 2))
 (segment (start 165.862 112.442) (end 165.862 107.442) (width 0.5) (layer "B.Cu") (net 18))
 (segment (start 137.922 112.442) (end 137.922 107.442) (width 0.5) (layer "B.Cu") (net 7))
 (segment (start 163.322 107.442) (end 163.322 112.442) (width 0.5) (layer "B.Cu") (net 17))
 (segment (start 177.8 124.9) (end 175.446 127.254) (width 0.5) (layer "F.Cu") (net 22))
 (segment (start 177.8 87.066) (end 177.8 124.9) (width 0.5) (layer "F.Cu") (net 22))
 (segment (start 175.446 127.254) (end 173.446 129.254) (width 0.5) (layer "F.Cu") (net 22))
 (segment (start 173.446 129.254) (end 141.662 129.254) (width 0.5) (layer "F.Cu") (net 22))
 (segment (start 130.16 76.9) (end 180.158 76.9) (width 0.5) (layer "F.Cu") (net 22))
 (segment (start 180.158 76.9) (end 184.062 80.804) (width 0.5) (layer "F.Cu") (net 22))
 (segment (start 141.662 129.254) (end 136.662 134.254) (width 0.5) (layer "F.Cu") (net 22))
 (segment (start 184.062 80.804) (end 177.8 87.066) (width 0.5) (layer "F.Cu") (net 22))
 (segment (start 127.762 74.502) (end 130.16 76.9) (width 0.5) (layer "F.Cu") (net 22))
 (segment (start 127.762 79.502) (end 127.762 74.502) (width 0.5) (layer "B.Cu") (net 22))
 (segment (start 155.702 112.442) (end 155.702 107.442) (width 0.5) (layer "B.Cu") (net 14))
 (segment (start 140.462 107.442) (end 140.462 112.442) (width 0.5) (layer "B.Cu") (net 8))
 (segment (start 160.782 112.442) (end 160.782 107.442) (width 0.5) (layer "B.Cu") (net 16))
 (segment (start 158.242 107.442) (end 158.242 112.442) (width 0.5) (layer "B.Cu") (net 15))
 (segment (start 143.002 79.502) (end 143.002 74.502) (width 0.5) (layer "B.Cu") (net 28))
 (segment (start 148.082 79.502) (end 148.082 74.502) (width 0.5) (layer "B.Cu") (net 30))
 (segment (start 158.242 79.502) (end 158.242 74.502) (width 0.5) (layer "B.Cu") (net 34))
 (segment (start 160.782 74.502) (end 160.782 79.502) (width 0.5) (layer "B.Cu") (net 35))
 (segment (start 150.622 112.442) (end 150.622 107.442) (width 0.5) (layer "B.Cu") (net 12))
 (segment (start 165.862 74.502) (end 165.862 79.502) (width 0.5) (layer "B.Cu") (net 37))
 (segment (start 125.222 74.502) (end 125.222 79.502) (width 0.5) (layer "B.Cu") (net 21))
 (segment (start 150.622 74.502) (end 150.622 79.502) (width 0.5) (layer "B.Cu") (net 31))
 (segment (start 127.762 112.442) (end 127.762 107.442) (width 0.5) (layer "B.Cu") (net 3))
 (segment (start 145.542 107.442) (end 145.542 112.442) (width 0.5) (layer "B.Cu") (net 10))
 (segment (start 130.302 74.502) (end 130.302 79.502) (width 0.5) (layer "B.Cu") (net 23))
 (segment (start 132.842 79.502) (end 132.842 74.502) (width 0.5) (layer "B.Cu") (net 24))
 (segment (start 137.922 79.502) (end 137.922 74.502) (width 0.5) (layer "B.Cu") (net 26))
 (segment (start 155.702 74.502) (end 155.702 79.502) (width 0.5) (layer "B.Cu") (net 33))
 (segment (start 139.822 128.554) (end 171.606 128.554) (width 0.5) (layer "F.Cu") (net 20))
 (segment (start 181.522 80.804) (end 178.318 77.6) (width 0.5) (layer "F.Cu") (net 20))
 (segment (start 125.78 77.6) (end 122.682 74.502) (width 0.5) (layer "F.Cu") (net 20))
 (segment (start 134.122 134.254) (end 139.822 128.554) (width 0.5) (layer "F.Cu") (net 20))
 (segment (start 177.1 123.06) (end 177.1 85.226) (width 0.5) (layer "F.Cu") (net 20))
 (segment (start 178.318 77.6) (end 125.78 77.6) (width 0.5) (layer "F.Cu") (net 20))
 (segment (start 171.606 128.554) (end 172.906 127.254) (width 0.5) (layer "F.Cu") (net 20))
 (segment (start 177.1 85.226) (end 181.522 80.804) (width 0.5) (layer "F.Cu") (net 20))
 (segment (start 172.906 127.254) (end 177.1 123.06) (width 0.5) (layer "F.Cu") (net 20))
 (segment (start 122.682 79.502) (end 122.682 74.502) (width 0.5) (layer "B.Cu") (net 20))
 (segment (start 148.082 112.442) (end 148.082 107.442) (width 0.5) (layer "B.Cu") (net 11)))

